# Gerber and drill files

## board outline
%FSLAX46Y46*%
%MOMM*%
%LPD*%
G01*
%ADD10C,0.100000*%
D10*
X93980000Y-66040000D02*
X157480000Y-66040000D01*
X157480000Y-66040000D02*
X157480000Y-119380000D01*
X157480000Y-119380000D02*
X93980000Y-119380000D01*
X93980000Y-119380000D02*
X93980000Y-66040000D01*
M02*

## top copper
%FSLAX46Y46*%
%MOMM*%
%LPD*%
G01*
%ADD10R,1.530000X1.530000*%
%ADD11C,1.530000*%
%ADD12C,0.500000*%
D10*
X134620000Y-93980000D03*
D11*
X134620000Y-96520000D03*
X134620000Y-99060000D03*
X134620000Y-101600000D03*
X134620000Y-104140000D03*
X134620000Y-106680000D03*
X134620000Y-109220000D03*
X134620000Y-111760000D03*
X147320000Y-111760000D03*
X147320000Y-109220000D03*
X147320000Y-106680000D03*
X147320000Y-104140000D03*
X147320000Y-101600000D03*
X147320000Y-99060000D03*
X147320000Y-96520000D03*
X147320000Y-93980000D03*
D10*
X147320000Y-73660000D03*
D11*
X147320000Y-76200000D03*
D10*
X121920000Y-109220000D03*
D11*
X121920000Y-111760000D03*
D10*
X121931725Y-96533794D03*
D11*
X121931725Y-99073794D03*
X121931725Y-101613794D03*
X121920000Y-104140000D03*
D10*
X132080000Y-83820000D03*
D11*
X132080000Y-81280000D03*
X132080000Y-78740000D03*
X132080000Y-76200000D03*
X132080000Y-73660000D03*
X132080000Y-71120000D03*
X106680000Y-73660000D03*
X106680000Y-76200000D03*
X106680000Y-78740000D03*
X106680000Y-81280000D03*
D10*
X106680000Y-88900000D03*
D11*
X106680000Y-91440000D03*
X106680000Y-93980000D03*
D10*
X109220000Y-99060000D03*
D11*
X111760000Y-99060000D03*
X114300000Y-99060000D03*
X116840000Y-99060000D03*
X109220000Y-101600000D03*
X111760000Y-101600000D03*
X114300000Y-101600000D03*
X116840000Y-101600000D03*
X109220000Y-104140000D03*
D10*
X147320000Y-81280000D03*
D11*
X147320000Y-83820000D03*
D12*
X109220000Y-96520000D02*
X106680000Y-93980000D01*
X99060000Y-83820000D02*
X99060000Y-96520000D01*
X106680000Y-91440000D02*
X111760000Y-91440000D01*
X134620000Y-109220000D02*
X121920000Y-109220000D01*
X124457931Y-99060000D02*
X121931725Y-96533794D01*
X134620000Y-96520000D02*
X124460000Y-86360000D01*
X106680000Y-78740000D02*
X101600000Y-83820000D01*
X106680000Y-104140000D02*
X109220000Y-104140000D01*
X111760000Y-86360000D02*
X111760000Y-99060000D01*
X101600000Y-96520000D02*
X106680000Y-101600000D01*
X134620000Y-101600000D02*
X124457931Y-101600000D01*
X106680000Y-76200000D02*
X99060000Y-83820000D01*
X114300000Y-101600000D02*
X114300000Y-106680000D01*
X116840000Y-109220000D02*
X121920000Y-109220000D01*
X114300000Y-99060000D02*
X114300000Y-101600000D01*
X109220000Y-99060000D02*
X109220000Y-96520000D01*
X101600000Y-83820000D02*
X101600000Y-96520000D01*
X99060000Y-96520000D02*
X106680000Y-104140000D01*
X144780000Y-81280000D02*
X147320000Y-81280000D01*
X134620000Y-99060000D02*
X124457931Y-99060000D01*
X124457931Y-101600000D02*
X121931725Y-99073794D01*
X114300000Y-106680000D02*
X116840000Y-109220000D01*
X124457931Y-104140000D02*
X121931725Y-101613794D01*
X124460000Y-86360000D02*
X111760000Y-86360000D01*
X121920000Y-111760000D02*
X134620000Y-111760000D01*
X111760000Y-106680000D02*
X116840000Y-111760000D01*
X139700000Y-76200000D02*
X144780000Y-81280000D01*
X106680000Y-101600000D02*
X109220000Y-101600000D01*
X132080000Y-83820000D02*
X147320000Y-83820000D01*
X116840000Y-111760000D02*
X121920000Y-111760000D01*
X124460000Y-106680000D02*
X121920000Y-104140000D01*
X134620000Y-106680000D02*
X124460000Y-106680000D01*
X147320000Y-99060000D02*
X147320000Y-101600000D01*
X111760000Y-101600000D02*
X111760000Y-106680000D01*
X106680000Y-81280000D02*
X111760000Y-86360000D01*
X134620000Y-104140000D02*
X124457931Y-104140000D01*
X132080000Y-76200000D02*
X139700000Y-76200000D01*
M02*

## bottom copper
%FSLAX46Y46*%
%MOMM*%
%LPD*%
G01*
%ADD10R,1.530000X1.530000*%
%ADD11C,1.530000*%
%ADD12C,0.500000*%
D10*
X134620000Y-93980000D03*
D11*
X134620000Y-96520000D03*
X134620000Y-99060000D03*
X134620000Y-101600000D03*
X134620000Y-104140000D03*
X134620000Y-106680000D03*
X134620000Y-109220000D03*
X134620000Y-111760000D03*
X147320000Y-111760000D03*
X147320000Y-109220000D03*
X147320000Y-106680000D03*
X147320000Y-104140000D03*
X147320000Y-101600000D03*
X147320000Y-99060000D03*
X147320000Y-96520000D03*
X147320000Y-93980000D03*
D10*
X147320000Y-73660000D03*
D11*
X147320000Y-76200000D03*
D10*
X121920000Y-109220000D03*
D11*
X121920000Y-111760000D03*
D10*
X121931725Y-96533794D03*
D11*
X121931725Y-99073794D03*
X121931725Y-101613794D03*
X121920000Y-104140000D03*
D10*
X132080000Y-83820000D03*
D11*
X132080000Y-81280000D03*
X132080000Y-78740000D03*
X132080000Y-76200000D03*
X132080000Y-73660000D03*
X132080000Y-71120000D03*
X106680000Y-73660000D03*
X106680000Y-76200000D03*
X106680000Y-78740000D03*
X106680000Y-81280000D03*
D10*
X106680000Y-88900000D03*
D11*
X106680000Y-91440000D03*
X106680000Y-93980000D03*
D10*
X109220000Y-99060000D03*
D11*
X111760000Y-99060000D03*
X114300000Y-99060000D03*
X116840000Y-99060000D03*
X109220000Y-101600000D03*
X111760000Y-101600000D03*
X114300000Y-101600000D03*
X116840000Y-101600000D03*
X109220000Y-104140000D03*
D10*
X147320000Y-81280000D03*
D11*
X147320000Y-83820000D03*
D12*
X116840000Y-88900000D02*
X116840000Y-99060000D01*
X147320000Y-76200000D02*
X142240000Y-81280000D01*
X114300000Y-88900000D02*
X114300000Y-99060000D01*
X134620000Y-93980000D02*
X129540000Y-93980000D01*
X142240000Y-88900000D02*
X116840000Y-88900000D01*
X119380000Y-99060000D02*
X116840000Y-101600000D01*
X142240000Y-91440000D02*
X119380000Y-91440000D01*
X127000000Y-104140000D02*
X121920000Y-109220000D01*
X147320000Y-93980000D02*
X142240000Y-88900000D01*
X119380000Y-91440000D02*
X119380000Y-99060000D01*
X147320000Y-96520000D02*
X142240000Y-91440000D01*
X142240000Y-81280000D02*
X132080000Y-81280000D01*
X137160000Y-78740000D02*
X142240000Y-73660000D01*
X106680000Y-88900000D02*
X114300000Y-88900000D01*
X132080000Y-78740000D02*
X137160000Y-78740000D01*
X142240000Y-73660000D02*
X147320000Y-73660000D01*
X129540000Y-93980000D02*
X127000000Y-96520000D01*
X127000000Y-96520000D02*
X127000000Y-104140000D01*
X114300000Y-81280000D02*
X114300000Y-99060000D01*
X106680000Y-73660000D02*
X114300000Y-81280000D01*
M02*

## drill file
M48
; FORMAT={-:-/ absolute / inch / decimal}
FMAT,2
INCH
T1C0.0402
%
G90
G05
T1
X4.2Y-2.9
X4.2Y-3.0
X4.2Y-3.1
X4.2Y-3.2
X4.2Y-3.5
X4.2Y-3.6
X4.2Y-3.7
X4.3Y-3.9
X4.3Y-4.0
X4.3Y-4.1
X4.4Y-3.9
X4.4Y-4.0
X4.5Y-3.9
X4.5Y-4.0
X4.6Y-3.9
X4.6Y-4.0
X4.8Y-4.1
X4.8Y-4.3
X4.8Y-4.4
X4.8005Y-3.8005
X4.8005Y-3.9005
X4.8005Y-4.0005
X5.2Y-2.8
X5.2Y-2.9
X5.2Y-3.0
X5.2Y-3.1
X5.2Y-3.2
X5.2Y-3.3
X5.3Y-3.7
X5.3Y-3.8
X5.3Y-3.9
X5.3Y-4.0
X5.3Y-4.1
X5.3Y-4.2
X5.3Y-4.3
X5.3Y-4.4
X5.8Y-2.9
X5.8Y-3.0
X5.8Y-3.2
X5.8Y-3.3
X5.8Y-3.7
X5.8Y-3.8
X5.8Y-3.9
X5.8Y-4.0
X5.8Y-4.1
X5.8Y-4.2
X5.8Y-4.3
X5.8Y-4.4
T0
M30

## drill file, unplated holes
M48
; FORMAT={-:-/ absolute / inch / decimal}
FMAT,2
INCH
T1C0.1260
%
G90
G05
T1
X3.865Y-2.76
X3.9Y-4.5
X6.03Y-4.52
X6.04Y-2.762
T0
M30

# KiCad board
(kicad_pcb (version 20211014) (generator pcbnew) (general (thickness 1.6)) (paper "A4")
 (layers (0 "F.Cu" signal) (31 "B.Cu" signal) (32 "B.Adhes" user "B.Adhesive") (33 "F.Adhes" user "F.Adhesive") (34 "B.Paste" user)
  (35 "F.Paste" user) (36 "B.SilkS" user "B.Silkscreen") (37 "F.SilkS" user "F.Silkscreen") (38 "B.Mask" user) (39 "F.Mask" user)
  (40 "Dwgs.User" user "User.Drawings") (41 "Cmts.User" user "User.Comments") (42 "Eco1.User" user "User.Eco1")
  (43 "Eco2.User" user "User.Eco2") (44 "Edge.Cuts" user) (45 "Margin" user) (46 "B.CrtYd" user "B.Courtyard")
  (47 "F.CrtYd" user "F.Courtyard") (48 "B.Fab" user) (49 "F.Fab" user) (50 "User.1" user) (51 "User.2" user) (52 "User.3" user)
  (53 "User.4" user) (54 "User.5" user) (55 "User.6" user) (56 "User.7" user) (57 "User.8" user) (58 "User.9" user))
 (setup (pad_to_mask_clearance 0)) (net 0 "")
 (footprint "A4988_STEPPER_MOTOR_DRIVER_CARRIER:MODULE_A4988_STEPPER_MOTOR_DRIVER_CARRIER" (layer "F.Cu") (at 140.97 102.87)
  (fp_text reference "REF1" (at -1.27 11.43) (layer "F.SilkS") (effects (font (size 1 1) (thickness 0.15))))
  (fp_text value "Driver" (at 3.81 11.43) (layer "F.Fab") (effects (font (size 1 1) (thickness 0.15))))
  (pad "1" thru_hole rect (at -6.35 -8.89) (size 1.53 1.53) (drill 1.02) (layers *.Cu *.Mask))
  (pad "2" thru_hole circle (at -6.35 -6.35) (size 1.53 1.53) (drill 1.02) (layers *.Cu *.Mask))
  (pad "3" thru_hole circle (at -6.35 -3.81) (size 1.53 1.53) (drill 1.02) (layers *.Cu *.Mask))
  (pad "4" thru_hole circle (at -6.35 -1.27) (size 1.53 1.53) (drill 1.02) (layers *.Cu *.Mask))
  (pad "5" thru_hole circle (at -6.35 1.27) (size 1.53 1.53) (drill 1.02) (layers *.Cu *.Mask))
  (pad "6" thru_hole circle (at -6.35 3.81) (size 1.53 1.53) (drill 1.02) (layers *.Cu *.Mask))
  (pad "7" thru_hole circle (at -6.35 6.35) (size 1.53 1.53) (drill 1.02) (layers *.Cu *.Mask))
  (pad "8" thru_hole circle (at -6.35 8.89) (size 1.53 1.53) (drill 1.02) (layers *.Cu *.Mask))
  (pad "9" thru_hole circle (at 6.35 8.89) (size 1.53 1.53) (drill 1.02) (layers *.Cu *.Mask))
  (pad "10" thru_hole circle (at 6.35 6.35) (size 1.53 1.53) (drill 1.02) (layers *.Cu *.Mask))
  (pad "11" thru_hole circle (at 6.35 3.81) (size 1.53 1.53) (drill 1.02) (layers *.Cu *.Mask))
  (pad "12" thru_hole circle (at 6.35 1.27) (size 1.53 1.53) (drill 1.02) (layers *.Cu *.Mask))
  (pad "13" thru_hole circle (at 6.35 -1.27) (size 1.53 1.53) (drill 1.02) (layers *.Cu *.Mask))
  (pad "14" thru_hole circle (at 6.35 -3.81) (size 1.53 1.53) (drill 1.02) (layers *.Cu *.Mask))
  (pad "15" thru_hole circle (at 6.35 -6.35) (size 1.53 1.53) (drill 1.02) (layers *.Cu *.Mask))
  (pad "16" thru_hole circle (at 6.35 -8.89) (size 1.53 1.53) (drill 1.02) (layers *.Cu *.Mask)))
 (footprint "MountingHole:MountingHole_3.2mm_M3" (layer "F.Cu") (at 153.416 70.1548)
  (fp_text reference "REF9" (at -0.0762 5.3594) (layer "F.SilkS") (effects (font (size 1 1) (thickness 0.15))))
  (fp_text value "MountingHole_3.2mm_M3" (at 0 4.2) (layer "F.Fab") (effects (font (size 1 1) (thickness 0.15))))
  (pad "" np_thru_hole circle (at 0 0) (size 3.2 3.2) (drill 3.2) (layers *.Cu *.Mask)))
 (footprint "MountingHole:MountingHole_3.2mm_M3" (layer "F.Cu") (at 153.162 114.808)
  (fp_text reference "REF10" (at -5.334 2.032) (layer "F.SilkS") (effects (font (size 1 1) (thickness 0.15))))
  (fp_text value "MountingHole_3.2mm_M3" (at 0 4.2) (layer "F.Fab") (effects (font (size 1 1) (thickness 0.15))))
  (pad "" np_thru_hole circle (at 0 0) (size 3.2 3.2) (drill 3.2) (layers *.Cu *.Mask)))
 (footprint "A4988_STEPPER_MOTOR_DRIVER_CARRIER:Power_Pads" (layer "F.Cu") (at 147.32 76.2)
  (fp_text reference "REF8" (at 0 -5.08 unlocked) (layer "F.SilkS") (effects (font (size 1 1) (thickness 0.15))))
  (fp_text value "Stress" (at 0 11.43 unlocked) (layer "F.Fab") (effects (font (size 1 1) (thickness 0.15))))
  (pad "1" thru_hole rect (at 0 -2.54) (size 1.53 1.53) (drill 1.02) (layers *.Cu *.Mask))
  (pad "2" thru_hole circle (at 0 0) (size 1.53 1.53) (drill 1.02) (layers *.Cu *.Mask)))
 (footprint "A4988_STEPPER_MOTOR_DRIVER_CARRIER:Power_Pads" (layer "F.Cu") (at 121.92 111.76)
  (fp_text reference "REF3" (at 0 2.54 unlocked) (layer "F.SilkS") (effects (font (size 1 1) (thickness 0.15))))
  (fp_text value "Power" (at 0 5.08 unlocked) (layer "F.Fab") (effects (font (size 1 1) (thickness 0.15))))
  (pad "1" thru_hole rect (at 0 -2.54) (size 1.53 1.53) (drill 1.02) (layers *.Cu *.Mask))
  (pad "2" thru_hole circle (at 0 0) (size 1.53 1.53) (drill 1.02) (layers *.Cu *.Mask)))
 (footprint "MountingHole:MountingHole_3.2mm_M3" (layer "F.Cu") (at 99.06 114.3)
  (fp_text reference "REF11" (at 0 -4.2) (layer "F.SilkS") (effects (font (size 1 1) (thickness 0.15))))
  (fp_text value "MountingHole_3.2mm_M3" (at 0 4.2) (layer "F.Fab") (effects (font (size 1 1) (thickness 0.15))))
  (pad "" np_thru_hole circle (at 0 0) (size 3.2 3.2) (drill 3.2) (layers *.Cu *.Mask)))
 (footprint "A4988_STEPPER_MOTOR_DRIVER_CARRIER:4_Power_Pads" (layer "F.Cu") (at 114.311725 91.453794)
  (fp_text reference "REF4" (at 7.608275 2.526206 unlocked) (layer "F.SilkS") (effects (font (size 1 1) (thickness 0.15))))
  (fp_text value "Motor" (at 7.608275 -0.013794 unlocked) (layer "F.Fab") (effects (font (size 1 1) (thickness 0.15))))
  (pad "1" thru_hole rect (at 7.62 5.08) (size 1.53 1.53) (drill 1.02) (layers *.Cu *.Mask))
  (pad "2" thru_hole circle (at 7.62 7.62) (size 1.53 1.53) (drill 1.02) (layers *.Cu *.Mask))
  (pad "3" thru_hole circle (at 7.62 10.16) (size 1.53 1.53) (drill 1.02) (layers *.Cu *.Mask))
  (pad "4" thru_hole circle (at 7.608275 12.686206) (size 1.53 1.53) (drill 1.02) (layers *.Cu *.Mask)))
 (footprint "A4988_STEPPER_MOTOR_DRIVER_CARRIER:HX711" (layer "F.Cu") (at 137.16 78.74 180)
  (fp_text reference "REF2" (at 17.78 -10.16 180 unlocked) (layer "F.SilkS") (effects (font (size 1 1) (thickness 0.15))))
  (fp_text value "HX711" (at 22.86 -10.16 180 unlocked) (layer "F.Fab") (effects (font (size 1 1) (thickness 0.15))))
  (pad "1" thru_hole rect (at 5.08 -5.08 180) (size 1.53 1.53) (drill 1.02) (layers *.Cu *.Mask))
  (pad "2" thru_hole circle (at 5.08 -2.54 180) (size 1.53 1.53) (drill 1.02) (layers *.Cu *.Mask))
  (pad "3" thru_hole circle (at 5.08 0 180) (size 1.53 1.53) (drill 1.02) (layers *.Cu *.Mask))
  (pad "4" thru_hole circle (at 5.08 2.54 180) (size 1.53 1.53) (drill 1.02) (layers *.Cu *.Mask))
  (pad "5" thru_hole circle (at 5.08 5.08 180) (size 1.53 1.53) (drill 1.02) (layers *.Cu *.Mask))
  (pad "6" thru_hole circle (at 5.08 7.62 180) (size 1.53 1.53) (drill 1.02) (layers *.Cu *.Mask))
  (pad "7" thru_hole circle (at 30.48 5.08 180) (size 1.53 1.53) (drill 1.02) (layers *.Cu *.Mask))
  (pad "8" thru_hole circle (at 30.48 2.54 180) (size 1.53 1.53) (drill 1.02) (layers *.Cu *.Mask))
  (pad "9" thru_hole circle (at 30.48 0 180) (size 1.53 1.53) (drill 1.02) (layers *.Cu *.Mask))
  (pad "10" thru_hole circle (at 30.48 -2.54 180) (size 1.53 1.53) (drill 1.02) (layers *.Cu *.Mask)))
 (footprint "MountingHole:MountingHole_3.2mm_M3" (layer "F.Cu") (at 98.171 70.104)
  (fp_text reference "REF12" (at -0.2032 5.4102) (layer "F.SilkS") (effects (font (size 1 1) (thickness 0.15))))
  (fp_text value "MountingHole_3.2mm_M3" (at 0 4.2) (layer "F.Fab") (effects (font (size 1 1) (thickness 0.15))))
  (pad "" np_thru_hole circle (at 0 0) (size 3.2 3.2) (drill 3.2) (layers *.Cu *.Mask)))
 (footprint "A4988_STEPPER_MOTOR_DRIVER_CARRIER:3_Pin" (layer "F.Cu") (at 106.68 88.9)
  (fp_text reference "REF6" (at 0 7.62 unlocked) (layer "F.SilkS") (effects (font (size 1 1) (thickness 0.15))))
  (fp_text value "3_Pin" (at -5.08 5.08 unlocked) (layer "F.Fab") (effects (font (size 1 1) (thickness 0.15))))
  (pad "1" thru_hole rect (at 0 0) (size 1.53 1.53) (drill 1.02) (layers *.Cu *.Mask))
  (pad "2" thru_hole circle (at 0 2.54) (size 1.53 1.53) (drill 1.02) (layers *.Cu *.Mask))
  (pad "3" thru_hole circle (at 0 5.08) (size 1.53 1.53) (drill 1.02) (layers *.Cu *.Mask)))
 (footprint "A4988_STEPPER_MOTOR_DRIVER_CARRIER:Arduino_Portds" (layer "F.Cu") (at 111.76 99.06)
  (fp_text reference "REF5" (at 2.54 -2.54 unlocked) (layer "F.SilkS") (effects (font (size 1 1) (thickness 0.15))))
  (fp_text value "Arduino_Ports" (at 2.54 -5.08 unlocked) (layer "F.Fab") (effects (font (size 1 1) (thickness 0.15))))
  (pad "1" thru_hole rect (at -2.54 0) (size 1.53 1.53) (drill 1.02) (layers *.Cu *.Mask))
  (pad "2" thru_hole circle (at 0 0) (size 1.53 1.53) (drill 1.02) (layers *.Cu *.Mask))
  (pad "3" thru_hole circle (at 2.54 0) (size 1.53 1.53) (drill 1.02) (layers *.Cu *.Mask))
  (pad "4" thru_hole circle (at 5.08 0) (size 1.53 1.53) (drill 1.02) (layers *.Cu *.Mask))
  (pad "5" thru_hole circle (at -2.54 2.54) (size 1.53 1.53) (drill 1.02) (layers *.Cu *.Mask))
  (pad "6" thru_hole circle (at 0 2.54) (size 1.53 1.53) (drill 1.02) (layers *.Cu *.Mask))
  (pad "7" thru_hole circle (at 2.54 2.54) (size 1.53 1.53) (drill 1.02) (layers *.Cu *.Mask))
  (pad "8" thru_hole circle (at 5.08 2.54) (size 1.53 1.53) (drill 1.02) (layers *.Cu *.Mask))
  (pad "9" thru_hole circle (at -2.54 5.08) (size 1.53 1.53) (drill 1.02) (layers *.Cu *.Mask)))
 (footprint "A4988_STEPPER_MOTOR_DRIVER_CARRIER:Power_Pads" (layer "F.Cu") (at 147.32 83.82)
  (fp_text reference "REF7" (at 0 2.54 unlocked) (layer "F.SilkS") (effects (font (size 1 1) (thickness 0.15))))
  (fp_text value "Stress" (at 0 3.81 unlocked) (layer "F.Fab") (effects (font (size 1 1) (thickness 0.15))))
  (pad "1" thru_hole rect (at 0 -2.54) (size 1.53 1.53) (drill 1.02) (layers *.Cu *.Mask))
  (pad "2" thru_hole circle (at 0 0) (size 1.53 1.53) (drill 1.02) (layers *.Cu *.Mask)))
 (gr_rect (start 93.98 66.04) (end 157.48 119.38) (layer "Edge.Cuts") (width 0.1) (fill none))
 (segment (start 109.22 96.52) (end 106.68 93.98) (width 0.5) (layer "F.Cu") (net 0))
 (segment (start 99.06 83.82) (end 99.06 96.52) (width 0.5) (layer "F.Cu") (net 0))
 (segment (start 106.68 91.44) (end 111.76 91.44) (width 0.5) (layer "F.Cu") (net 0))
 (segment (start 134.62 109.22) (end 121.92 109.22) (width 0.5) (layer "F.Cu") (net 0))
 (segment (start 124.457931 99.06) (end 121.931725 96.533794) (width 0.5) (layer "F.Cu") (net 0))
 (segment (start 134.62 96.52) (end 124.46 86.36) (width 0.5) (layer "F.Cu") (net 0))
 (segment (start 106.68 78.74) (end 101.6 83.82) (width 0.5) (layer "F.Cu") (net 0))
 (segment (start 106.68 104.14) (end 109.22 104.14) (width 0.5) (layer "F.Cu") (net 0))
 (segment (start 111.76 86.36) (end 111.76 99.06) (width 0.5) (layer "F.Cu") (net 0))
 (segment (start 101.6 96.52) (end 106.68 101.6) (width 0.5) (layer "F.Cu") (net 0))
 (segment (start 134.62 101.6) (end 124.457931 101.6) (width 0.5) (layer "F.Cu") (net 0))
 (segment (start 106.68 76.2) (end 99.06 83.82) (width 0.5) (layer "F.Cu") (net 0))
 (segment (start 114.3 101.6) (end 114.3 106.68) (width 0.5) (layer "F.Cu") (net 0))
 (segment (start 116.84 109.22) (end 121.92 109.22) (width 0.5) (layer "F.Cu") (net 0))
 (segment (start 114.3 99.06) (end 114.3 101.6) (width 0.5) (layer "F.Cu") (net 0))
 (segment (start 109.22 99.06) (end 109.22 96.52) (width 0.5) (layer "F.Cu") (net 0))
 (segment (start 101.6 83.82) (end 101.6 96.52) (width 0.5) (layer "F.Cu") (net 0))
 (segment (start 99.06 96.52) (end 106.68 104.14) (width 0.5) (layer "F.Cu") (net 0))
 (segment (start 144.78 81.28) (end 147.32 81.28) (width 0.5) (layer "F.Cu") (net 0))
 (segment (start 134.62 99.06) (end 124.457931 99.06) (width 0.5) (layer "F.Cu") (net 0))
 (segment (start 124.457931 101.6) (end 121.931725 99.073794) (width 0.5) (layer "F.Cu") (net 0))
 (segment (start 114.3 106.68) (end 116.84 109.22) (width 0.5) (layer "F.Cu") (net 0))
 (segment (start 124.457931 104.14) (end 121.931725 101.613794) (width 0.5) (layer "F.Cu") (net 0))
 (segment (start 124.46 86.36) (end 111.76 86.36) (width 0.5) (layer "F.Cu") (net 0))
 (segment (start 121.92 111.76) (end 134.62 111.76) (width 0.5) (layer "F.Cu") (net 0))
 (segment (start 111.76 106.68) (end 116.84 111.76) (width 0.5) (layer "F.Cu") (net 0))
 (segment (start 139.7 76.2) (end 144.78 81.28) (width 0.5) (layer "F.Cu") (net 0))
 (segment (start 106.68 101.6) (end 109.22 101.6) (width 0.5) (layer "F.Cu") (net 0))
 (segment (start 132.08 83.82) (end 147.32 83.82) (width 0.5) (layer "F.Cu") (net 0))
 (segment (start 116.84 111.76) (end 121.92 111.76) (width 0.5) (layer "F.Cu") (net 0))
 (segment (start 124.46 106.68) (end 121.92 104.14) (width 0.5) (layer "F.Cu") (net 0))
 (segment (start 134.62 106.68) (end 124.46 106.68) (width 0.5) (layer "F.Cu") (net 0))
 (segment (start 147.32 99.06) (end 147.32 101.6) (width 0.5) (layer "F.Cu") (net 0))
 (segment (start 111.76 101.6) (end 111.76 106.68) (width 0.5) (layer "F.Cu") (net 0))
 (segment (start 106.68 81.28) (end 111.76 86.36) (width 0.5) (layer "F.Cu") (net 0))
 (segment (start 134.62 104.14) (end 124.457931 104.14) (width 0.5) (layer "F.Cu") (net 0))
 (segment (start 132.08 76.2) (end 139.7 76.2) (width 0.5) (layer "F.Cu") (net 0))
 (segment (start 116.84 88.9) (end 116.84 99.06) (width 0.5) (layer "B.Cu") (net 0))
 (segment (start 147.32 76.2) (end 142.24 81.28) (width 0.5) (layer "B.Cu") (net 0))
 (segment (start 114.3 88.9) (end 114.3 99.06) (width 0.5) (layer "B.Cu") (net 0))
 (segment (start 134.62 93.98) (end 129.54 93.98) (width 0.5) (layer "B.Cu") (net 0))
 (segment (start 142.24 88.9) (end 116.84 88.9) (width 0.5) (layer "B.Cu") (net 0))
 (segment (start 119.38 99.06) (end 116.84 101.6) (width 0.5) (layer "B.Cu") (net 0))
 (segment (start 142.24 91.44) (end 119.38 91.44) (width 0.5) (layer "B.Cu") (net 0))
 (segment (start 127 104.14) (end 121.92 109.22) (width 0.5) (layer "B.Cu") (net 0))
 (segment (start 147.32 93.98) (end 142.24 88.9) (width 0.5) (layer "B.Cu") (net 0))
 (segment (start 119.38 91.44) (end 119.38 99.06) (width 0.5) (layer "B.Cu") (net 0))
 (segment (start 147.32 96.52) (end 142.24 91.44) (width 0.5) (layer "B.Cu") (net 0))
 (segment (start 142.24 81.28) (end 132.08 81.28) (width 0.5) (layer "B.Cu") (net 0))
 (segment (start 137.16 78.74) (end 142.24 73.66) (width 0.5) (layer "B.Cu") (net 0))
 (segment (start 106.68 88.9) (end 114.3 88.9) (width 0.5) (layer "B.Cu") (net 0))
 (segment (start 132.08 78.74) (end 137.16 78.74) (width 0.5) (layer "B.Cu") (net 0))
 (segment (start 142.24 73.66) (end 147.32 73.66) (width 0.5) (layer "B.Cu") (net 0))
 (segment (start 129.54 93.98) (end 127 96.52) (width 0.5) (layer "B.Cu") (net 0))
 (segment (start 127 96.52) (end 127 104.14) (width 0.5) (layer "B.Cu") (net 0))
 (segment (start 114.3 81.28) (end 114.3 99.06) (width 0.5) (layer "B.Cu") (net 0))
 (segment (start 106.68 73.66) (end 114.3 81.28) (width 0.5) (layer "B.Cu") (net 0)))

